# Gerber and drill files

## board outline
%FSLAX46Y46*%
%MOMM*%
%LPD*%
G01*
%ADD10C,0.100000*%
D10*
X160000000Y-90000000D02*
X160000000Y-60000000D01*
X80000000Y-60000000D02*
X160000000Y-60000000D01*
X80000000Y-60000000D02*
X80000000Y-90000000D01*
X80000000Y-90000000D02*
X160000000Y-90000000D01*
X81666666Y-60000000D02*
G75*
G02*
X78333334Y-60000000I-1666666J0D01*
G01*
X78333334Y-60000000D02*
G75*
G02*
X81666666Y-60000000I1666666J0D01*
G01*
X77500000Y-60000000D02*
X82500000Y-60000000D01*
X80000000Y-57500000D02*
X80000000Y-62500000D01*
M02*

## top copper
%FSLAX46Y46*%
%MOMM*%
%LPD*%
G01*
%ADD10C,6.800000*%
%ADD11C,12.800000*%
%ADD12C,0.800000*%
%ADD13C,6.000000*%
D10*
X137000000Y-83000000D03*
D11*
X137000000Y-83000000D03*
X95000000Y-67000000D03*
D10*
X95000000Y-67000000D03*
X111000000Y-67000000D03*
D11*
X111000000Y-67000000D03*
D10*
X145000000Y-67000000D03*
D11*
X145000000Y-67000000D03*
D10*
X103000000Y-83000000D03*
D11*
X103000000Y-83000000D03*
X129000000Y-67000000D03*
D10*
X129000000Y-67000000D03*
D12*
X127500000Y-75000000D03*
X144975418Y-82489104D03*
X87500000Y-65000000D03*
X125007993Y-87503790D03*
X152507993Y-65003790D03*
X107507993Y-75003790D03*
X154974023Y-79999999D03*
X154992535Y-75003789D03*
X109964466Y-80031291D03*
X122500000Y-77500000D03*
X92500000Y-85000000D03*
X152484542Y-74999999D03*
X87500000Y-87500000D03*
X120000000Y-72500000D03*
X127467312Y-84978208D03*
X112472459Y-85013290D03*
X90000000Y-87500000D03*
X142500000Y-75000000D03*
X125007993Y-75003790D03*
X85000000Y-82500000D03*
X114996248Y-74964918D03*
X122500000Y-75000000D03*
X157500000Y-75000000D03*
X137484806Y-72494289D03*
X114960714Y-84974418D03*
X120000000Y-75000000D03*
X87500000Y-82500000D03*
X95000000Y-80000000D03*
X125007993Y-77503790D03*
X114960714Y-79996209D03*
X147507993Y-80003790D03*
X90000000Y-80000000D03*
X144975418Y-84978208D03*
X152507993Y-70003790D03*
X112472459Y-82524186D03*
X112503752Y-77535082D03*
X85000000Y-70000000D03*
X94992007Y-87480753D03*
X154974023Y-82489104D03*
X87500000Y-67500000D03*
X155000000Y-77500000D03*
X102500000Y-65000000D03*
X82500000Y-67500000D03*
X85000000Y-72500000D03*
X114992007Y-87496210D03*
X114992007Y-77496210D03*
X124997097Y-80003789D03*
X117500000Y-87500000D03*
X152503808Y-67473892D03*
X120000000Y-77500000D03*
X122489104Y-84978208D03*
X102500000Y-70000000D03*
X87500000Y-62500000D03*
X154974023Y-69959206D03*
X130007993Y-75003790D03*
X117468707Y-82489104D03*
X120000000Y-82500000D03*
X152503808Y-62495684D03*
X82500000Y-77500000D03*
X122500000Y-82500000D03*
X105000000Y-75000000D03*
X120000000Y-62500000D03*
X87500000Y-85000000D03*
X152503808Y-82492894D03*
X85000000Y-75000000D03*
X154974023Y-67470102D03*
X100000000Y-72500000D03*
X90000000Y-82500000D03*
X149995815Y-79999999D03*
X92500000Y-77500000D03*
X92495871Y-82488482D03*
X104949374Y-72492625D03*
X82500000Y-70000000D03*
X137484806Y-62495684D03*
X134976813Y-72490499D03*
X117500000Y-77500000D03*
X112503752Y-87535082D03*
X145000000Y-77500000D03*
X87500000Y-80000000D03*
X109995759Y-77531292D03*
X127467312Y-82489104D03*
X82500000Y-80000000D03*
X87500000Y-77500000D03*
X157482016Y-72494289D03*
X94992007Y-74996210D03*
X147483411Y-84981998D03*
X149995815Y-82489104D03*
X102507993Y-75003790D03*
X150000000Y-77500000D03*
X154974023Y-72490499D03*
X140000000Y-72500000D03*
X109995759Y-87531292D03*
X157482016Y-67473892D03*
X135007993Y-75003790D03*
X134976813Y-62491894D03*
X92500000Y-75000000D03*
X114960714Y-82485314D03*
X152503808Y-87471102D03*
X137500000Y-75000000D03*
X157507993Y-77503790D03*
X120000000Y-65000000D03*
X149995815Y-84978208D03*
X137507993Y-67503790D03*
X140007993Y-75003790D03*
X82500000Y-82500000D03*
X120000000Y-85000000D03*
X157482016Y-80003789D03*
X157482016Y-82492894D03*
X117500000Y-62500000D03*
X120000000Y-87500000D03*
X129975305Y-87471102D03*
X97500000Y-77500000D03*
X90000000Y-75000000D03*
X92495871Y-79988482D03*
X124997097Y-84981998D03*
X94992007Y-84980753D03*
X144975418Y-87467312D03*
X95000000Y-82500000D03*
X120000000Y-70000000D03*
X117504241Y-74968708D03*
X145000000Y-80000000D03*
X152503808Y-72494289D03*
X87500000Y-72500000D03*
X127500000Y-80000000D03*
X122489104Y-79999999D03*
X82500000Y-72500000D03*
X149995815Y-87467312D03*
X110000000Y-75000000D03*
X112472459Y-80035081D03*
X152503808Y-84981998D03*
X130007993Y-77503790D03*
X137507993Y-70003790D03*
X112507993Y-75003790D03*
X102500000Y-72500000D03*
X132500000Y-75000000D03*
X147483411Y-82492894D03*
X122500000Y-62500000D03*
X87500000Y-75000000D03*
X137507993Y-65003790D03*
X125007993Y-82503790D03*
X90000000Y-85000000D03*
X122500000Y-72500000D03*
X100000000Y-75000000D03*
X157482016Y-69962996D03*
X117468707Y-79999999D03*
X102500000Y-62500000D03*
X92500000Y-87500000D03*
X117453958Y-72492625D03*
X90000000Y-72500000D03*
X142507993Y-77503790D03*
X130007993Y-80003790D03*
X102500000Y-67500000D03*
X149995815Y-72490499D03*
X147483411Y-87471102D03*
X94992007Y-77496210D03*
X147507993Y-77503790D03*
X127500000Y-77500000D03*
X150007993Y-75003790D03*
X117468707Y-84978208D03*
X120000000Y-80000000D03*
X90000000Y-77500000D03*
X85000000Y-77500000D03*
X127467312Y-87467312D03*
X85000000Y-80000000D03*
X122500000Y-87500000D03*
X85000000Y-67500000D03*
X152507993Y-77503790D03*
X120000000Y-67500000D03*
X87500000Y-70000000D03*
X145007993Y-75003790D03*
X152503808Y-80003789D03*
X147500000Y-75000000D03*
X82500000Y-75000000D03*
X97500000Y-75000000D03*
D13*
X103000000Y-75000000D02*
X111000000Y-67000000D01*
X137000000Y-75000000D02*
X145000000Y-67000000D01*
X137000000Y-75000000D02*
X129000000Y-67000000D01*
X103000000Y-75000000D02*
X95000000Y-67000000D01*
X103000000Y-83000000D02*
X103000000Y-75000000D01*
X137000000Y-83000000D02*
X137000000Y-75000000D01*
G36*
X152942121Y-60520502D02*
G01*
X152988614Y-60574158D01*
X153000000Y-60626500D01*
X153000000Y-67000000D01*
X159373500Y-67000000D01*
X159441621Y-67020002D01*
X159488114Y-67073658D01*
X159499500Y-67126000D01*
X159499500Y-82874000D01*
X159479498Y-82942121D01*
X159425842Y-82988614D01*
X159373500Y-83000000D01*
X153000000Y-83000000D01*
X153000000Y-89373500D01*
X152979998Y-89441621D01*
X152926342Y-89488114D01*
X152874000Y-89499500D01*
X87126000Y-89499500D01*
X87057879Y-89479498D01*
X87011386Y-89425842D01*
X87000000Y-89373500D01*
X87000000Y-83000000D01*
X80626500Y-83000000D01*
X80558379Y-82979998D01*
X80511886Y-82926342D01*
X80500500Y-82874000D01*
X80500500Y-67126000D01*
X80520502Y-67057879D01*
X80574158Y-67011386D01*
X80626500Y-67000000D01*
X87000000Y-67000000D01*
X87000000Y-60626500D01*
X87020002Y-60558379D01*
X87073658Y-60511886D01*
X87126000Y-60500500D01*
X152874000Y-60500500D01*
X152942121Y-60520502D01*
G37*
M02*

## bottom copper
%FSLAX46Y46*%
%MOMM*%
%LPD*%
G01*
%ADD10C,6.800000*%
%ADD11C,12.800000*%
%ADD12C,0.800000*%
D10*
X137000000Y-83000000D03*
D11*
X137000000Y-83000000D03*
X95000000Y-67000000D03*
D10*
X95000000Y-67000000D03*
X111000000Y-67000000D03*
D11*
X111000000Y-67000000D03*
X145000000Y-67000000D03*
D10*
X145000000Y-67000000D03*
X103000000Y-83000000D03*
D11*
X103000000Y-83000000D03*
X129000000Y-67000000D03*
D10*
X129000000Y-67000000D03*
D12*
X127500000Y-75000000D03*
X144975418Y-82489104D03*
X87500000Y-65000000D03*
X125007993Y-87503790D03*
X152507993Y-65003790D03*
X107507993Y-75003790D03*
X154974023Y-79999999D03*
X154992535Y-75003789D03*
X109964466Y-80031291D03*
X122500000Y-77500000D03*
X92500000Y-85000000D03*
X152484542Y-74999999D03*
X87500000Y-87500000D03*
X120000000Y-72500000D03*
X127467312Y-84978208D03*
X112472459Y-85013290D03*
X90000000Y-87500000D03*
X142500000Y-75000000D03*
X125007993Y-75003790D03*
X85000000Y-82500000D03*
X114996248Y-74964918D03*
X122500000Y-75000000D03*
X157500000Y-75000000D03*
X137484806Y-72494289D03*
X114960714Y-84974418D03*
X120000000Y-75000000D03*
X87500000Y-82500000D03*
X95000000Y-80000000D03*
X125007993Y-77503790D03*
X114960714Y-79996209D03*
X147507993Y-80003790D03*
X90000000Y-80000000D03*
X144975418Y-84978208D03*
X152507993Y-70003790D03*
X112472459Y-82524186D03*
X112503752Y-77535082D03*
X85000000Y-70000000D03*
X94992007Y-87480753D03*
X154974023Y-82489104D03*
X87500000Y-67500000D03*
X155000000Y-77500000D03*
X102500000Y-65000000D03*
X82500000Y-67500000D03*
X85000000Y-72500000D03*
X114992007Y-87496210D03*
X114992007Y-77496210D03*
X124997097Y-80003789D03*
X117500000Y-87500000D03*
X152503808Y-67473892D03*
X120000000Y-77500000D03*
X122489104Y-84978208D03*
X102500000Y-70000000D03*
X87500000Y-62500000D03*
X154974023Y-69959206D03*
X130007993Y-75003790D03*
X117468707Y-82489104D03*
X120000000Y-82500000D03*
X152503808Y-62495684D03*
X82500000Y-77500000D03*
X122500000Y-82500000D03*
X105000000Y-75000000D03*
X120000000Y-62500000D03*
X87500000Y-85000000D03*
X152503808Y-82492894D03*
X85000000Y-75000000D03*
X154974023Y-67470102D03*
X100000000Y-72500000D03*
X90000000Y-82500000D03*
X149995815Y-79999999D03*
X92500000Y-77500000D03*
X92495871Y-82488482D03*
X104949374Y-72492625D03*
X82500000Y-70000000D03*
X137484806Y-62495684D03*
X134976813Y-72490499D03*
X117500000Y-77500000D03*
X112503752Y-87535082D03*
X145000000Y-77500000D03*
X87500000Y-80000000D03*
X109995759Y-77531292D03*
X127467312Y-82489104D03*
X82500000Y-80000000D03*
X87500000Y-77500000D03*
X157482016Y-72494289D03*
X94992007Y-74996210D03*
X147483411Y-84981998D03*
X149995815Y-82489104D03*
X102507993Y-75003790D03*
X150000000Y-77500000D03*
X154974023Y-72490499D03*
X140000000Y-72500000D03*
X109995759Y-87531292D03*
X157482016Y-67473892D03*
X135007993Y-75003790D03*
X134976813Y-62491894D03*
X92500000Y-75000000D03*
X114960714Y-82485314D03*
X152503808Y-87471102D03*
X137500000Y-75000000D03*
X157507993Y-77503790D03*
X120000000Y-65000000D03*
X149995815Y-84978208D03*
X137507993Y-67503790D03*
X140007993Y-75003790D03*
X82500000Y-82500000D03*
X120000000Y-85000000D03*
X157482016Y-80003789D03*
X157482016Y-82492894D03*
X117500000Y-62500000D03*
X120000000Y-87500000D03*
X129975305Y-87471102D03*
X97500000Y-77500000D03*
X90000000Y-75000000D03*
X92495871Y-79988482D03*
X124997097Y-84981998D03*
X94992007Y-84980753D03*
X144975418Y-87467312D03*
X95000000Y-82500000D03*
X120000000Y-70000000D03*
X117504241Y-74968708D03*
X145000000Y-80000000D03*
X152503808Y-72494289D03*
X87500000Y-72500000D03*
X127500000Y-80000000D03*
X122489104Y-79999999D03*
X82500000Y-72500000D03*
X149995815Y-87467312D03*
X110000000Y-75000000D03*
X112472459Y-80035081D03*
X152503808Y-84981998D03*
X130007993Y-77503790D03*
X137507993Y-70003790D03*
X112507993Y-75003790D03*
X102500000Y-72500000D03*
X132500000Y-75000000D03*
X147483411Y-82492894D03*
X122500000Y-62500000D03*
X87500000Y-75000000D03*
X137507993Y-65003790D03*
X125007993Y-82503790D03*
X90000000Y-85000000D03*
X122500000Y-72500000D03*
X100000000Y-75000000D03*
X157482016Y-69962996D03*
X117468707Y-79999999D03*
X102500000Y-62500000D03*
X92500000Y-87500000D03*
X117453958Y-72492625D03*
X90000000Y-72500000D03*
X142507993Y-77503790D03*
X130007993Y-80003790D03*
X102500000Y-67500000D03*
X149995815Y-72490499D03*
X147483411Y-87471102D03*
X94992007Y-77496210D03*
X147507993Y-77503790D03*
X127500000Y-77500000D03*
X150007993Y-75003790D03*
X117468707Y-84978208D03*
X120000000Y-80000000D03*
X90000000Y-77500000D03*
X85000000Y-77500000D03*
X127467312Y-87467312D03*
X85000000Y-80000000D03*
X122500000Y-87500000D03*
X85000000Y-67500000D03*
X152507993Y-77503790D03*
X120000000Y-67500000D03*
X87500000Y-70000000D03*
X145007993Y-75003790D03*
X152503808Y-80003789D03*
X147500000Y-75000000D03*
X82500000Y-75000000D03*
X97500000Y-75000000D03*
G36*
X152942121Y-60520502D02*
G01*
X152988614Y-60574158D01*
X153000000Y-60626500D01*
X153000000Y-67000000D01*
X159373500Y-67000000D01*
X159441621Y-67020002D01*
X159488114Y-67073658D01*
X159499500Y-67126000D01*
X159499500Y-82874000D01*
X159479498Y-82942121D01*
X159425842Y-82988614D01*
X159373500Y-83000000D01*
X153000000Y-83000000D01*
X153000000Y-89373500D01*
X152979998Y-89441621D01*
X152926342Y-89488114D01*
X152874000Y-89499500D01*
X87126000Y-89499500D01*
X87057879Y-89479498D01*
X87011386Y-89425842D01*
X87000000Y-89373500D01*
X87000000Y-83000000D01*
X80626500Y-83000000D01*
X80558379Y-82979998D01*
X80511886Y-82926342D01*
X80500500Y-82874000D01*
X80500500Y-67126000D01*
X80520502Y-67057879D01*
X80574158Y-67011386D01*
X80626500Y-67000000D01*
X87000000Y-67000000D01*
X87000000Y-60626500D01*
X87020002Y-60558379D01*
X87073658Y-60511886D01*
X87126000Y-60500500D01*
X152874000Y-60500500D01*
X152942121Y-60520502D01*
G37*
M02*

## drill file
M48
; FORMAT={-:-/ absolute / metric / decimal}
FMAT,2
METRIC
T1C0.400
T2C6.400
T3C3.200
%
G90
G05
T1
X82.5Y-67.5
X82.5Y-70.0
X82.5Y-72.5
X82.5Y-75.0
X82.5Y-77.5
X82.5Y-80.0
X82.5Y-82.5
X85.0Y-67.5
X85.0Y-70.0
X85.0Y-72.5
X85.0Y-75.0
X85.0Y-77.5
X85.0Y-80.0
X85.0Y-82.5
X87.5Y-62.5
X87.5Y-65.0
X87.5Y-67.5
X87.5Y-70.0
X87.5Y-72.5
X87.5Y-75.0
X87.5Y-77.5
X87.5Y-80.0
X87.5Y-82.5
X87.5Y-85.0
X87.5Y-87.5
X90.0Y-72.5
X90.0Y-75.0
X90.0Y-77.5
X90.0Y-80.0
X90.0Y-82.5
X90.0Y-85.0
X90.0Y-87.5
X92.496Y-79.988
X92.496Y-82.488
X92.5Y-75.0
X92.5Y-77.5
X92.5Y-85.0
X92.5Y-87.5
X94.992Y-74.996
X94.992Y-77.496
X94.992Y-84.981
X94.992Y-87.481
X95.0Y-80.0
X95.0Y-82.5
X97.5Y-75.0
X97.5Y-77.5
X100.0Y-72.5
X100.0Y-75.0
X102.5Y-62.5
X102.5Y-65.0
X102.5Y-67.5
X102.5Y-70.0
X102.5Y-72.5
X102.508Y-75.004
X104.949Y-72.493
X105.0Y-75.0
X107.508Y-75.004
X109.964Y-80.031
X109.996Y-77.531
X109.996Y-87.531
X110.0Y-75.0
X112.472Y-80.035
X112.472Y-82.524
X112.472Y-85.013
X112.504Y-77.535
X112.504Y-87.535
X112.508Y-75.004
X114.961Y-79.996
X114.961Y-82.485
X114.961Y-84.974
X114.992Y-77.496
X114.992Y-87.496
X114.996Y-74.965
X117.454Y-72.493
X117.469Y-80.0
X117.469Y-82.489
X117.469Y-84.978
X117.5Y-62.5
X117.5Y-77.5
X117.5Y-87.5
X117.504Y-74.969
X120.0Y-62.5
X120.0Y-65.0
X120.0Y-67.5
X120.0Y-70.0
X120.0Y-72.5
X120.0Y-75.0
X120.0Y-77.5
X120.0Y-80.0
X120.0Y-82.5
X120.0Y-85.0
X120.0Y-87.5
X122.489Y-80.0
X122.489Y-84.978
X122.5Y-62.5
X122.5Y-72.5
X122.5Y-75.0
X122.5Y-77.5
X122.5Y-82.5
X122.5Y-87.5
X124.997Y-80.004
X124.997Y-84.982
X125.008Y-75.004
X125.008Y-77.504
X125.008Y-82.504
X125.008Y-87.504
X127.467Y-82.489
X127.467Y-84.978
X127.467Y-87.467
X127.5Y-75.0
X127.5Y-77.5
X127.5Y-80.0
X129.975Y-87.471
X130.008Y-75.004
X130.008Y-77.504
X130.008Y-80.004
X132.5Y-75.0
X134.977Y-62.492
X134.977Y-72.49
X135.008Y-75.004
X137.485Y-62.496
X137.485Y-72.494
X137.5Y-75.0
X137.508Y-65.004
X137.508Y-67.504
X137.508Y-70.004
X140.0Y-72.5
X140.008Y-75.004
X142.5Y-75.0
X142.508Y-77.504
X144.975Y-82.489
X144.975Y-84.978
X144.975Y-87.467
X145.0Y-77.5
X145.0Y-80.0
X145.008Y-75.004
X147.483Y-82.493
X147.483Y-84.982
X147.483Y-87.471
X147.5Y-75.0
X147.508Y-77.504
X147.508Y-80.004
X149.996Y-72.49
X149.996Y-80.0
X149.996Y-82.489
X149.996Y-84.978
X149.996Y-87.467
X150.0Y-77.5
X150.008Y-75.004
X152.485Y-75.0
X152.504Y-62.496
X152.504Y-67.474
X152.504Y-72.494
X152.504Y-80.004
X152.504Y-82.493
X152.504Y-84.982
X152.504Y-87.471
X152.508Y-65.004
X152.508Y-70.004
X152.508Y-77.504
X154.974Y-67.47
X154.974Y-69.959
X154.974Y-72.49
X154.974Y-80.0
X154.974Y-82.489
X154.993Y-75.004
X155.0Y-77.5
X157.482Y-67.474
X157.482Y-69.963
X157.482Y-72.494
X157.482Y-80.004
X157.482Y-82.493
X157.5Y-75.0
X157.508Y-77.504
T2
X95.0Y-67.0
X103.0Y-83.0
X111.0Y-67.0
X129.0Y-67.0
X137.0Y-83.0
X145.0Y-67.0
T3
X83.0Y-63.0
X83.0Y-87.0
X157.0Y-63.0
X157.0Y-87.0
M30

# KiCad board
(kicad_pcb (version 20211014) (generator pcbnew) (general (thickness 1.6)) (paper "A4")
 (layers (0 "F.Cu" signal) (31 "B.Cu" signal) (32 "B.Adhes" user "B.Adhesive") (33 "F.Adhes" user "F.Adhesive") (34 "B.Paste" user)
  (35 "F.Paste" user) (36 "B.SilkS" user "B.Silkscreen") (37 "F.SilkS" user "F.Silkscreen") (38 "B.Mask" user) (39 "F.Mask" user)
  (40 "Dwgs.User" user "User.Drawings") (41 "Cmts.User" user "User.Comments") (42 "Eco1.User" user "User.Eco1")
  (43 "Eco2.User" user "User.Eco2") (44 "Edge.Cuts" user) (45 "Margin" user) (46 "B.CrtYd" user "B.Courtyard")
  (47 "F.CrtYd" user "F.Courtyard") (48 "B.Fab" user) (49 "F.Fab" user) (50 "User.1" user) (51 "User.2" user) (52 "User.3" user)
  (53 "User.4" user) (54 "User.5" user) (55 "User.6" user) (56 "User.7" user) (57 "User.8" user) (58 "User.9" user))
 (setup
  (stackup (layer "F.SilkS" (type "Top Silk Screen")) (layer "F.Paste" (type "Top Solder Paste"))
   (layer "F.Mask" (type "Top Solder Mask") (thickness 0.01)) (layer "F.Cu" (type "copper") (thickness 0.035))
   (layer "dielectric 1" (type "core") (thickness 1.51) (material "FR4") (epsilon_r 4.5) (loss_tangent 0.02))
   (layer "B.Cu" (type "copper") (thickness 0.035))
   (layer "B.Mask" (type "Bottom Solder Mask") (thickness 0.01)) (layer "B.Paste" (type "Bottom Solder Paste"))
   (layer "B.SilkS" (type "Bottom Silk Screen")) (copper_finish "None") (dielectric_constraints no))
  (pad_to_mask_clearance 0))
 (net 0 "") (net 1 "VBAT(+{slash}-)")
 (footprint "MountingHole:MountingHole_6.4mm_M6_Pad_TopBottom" (layer "F.Cu") (at 137 83 90)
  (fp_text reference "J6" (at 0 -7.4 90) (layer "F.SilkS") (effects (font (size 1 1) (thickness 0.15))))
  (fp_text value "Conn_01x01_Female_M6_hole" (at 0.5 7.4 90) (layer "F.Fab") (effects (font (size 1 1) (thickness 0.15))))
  (pad "1" thru_hole circle locked (at 0 0 90) (size 6.8 6.8) (drill 6.4) (layers *.Cu *.Mask) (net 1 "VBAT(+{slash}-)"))
  (pad "1" connect circle locked (at 0 0 90) (size 12.8 12.8) (layers "F.Cu" "F.Mask") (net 1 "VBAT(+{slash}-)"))
  (pad "1" connect circle locked (at 0 0 90) (size 12.8 12.8) (layers "B.Cu" "B.Mask") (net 1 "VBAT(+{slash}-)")))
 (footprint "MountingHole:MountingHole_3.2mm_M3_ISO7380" (layer "F.Cu") (at 157 87)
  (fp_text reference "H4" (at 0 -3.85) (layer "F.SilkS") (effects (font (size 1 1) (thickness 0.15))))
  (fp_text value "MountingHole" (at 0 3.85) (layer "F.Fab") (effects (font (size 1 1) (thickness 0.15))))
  (pad "" np_thru_hole circle locked (at 0 0) (size 3.2 3.2) (drill 3.2) (layers *.Cu *.Mask)))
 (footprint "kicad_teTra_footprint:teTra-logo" (layer "F.Cu") (at 86 75)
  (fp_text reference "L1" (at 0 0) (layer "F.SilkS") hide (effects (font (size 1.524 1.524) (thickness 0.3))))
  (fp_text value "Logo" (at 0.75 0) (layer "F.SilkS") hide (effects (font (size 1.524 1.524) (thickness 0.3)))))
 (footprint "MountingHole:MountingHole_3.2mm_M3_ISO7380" (layer "F.Cu") (at 83 87)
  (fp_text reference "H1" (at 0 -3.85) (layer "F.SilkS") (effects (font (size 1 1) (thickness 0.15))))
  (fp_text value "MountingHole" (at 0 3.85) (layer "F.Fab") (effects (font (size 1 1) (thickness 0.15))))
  (pad "" np_thru_hole circle locked (at 0 0) (size 3.2 3.2) (drill 3.2) (layers *.Cu *.Mask)))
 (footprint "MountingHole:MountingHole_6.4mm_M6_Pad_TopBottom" (layer "F.Cu") (at 95 67 90)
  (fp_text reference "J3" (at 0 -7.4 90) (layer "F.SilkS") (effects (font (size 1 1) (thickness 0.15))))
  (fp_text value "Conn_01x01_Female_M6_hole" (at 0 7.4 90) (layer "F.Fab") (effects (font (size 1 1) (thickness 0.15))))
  (pad "1" connect circle locked (at 0 0 90) (size 12.8 12.8) (layers "B.Cu" "B.Mask") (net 1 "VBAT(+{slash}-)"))
  (pad "1" connect circle locked (at 0 0 90) (size 12.8 12.8) (layers "F.Cu" "F.Mask") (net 1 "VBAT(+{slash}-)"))
  (pad "1" thru_hole circle locked (at 0 0 90) (size 6.8 6.8) (drill 6.4) (layers *.Cu *.Mask) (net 1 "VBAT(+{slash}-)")))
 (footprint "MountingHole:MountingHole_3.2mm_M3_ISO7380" (layer "F.Cu") (at 83 63)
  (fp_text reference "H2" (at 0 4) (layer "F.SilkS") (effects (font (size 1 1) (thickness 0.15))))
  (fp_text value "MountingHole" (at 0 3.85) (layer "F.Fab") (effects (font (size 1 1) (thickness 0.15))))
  (pad "" np_thru_hole circle locked (at 0 0) (size 3.2 3.2) (drill 3.2) (layers *.Cu *.Mask)))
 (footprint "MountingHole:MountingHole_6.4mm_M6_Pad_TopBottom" (layer "F.Cu") (at 111 67 90)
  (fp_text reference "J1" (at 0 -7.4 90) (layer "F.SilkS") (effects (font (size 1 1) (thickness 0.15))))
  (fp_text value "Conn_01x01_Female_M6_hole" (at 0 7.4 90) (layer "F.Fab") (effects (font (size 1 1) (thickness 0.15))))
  (pad "1" thru_hole circle locked (at 0 0 90) (size 6.8 6.8) (drill 6.4) (layers *.Cu *.Mask) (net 1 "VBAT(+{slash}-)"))
  (pad "1" connect circle locked (at 0 0 90) (size 12.8 12.8) (layers "F.Cu" "F.Mask") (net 1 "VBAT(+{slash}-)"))
  (pad "1" connect circle locked (at 0 0 90) (size 12.8 12.8) (layers "B.Cu" "B.Mask") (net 1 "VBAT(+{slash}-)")))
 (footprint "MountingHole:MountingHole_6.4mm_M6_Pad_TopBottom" (layer "F.Cu") (at 145 67 90)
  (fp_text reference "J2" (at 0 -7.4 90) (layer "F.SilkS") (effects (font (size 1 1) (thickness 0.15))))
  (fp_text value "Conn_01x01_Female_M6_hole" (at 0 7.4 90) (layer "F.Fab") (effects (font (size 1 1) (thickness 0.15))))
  (pad "1" connect circle locked (at 0 0 90) (size 12.8 12.8) (layers "B.Cu" "B.Mask") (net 1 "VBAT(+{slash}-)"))
  (pad "1" thru_hole circle locked (at 0 0 90) (size 6.8 6.8) (drill 6.4) (layers *.Cu *.Mask) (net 1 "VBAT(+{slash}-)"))
  (pad "1" connect circle locked (at 0 0 90) (size 12.8 12.8) (layers "F.Cu" "F.Mask") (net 1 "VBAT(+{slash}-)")))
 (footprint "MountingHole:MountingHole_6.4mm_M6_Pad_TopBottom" (layer "F.Cu") (at 103 83 90)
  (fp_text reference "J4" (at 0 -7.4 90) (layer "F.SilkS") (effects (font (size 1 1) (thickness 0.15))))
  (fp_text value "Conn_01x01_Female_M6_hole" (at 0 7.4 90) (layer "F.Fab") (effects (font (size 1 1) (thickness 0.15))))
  (pad "1" thru_hole circle locked (at 0 0 90) (size 6.8 6.8) (drill 6.4) (layers *.Cu *.Mask) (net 1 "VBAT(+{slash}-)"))
  (pad "1" connect circle locked (at 0 0 90) (size 12.8 12.8) (layers "B.Cu" "B.Mask") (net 1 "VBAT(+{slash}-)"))
  (pad "1" connect circle locked (at 0 0 90) (size 12.8 12.8) (layers "F.Cu" "F.Mask") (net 1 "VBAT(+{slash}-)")))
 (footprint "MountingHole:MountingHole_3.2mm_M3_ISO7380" (layer "F.Cu") (at 157 63)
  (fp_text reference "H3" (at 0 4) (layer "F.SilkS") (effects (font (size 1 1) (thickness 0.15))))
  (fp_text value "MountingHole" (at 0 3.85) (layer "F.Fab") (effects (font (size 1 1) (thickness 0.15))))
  (pad "" np_thru_hole circle locked (at 0 0) (size 3.2 3.2) (drill 3.2) (layers *.Cu *.Mask)))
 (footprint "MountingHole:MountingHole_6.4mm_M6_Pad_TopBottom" (layer "F.Cu") (at 129 67 90)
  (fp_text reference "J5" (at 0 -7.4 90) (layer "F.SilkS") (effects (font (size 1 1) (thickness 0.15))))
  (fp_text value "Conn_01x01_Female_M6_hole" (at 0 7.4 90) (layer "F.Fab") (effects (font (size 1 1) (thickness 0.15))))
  (pad "1" connect circle locked (at 0 0 90) (size 12.8 12.8) (layers "F.Cu" "F.Mask") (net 1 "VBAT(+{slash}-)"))
  (pad "1" connect circle locked (at 0 0 90) (size 12.8 12.8) (layers "B.Cu" "B.Mask") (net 1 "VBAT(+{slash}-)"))
  (pad "1" thru_hole circle locked (at 0 0 90) (size 6.8 6.8) (drill 6.4) (layers *.Cu *.Mask) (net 1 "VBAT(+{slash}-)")))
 (gr_line (start 160 90) (end 160 60) (layer "Edge.Cuts") (width 0.1))
 (gr_line (start 80 60) (end 160 60) (layer "Edge.Cuts") (width 0.1))
 (gr_line (start 80 60) (end 80 90) (layer "Edge.Cuts") (width 0.1))
 (gr_line (start 80 90) (end 160 90) (layer "Edge.Cuts") (width 0.1))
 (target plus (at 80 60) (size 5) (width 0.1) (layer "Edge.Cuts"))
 (segment (start 103 75) (end 111 67) (width 6) (layer "F.Cu") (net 1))
 (segment (start 137 75) (end 145 67) (width 6) (layer "F.Cu") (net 1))
 (segment (start 137 75) (end 129 67) (width 6) (layer "F.Cu") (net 1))
 (segment (start 103 75) (end 95 67) (width 6) (layer "F.Cu") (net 1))
 (segment (start 103 83) (end 103 75) (width 6) (layer "F.Cu") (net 1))
 (segment (start 137 83) (end 137 75) (width 6) (layer "F.Cu") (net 1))
 (via (at 127.5 75) (size 0.8) (drill 0.4) (layers "F.Cu" "B.Cu") (free) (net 1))
 (via (at 144.975418 82.489104) (size 0.8) (drill 0.4) (layers "F.Cu" "B.Cu") (free) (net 1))
 (via (at 87.5 65) (size 0.8) (drill 0.4) (layers "F.Cu" "B.Cu") (free) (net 1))
 (via (at 125.007993 87.50379) (size 0.8) (drill 0.4) (layers "F.Cu" "B.Cu") (free) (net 1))
 (via (at 152.507993 65.00379) (size 0.8) (drill 0.4) (layers "F.Cu" "B.Cu") (free) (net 1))
 (via (at 107.507993 75.00379) (size 0.8) (drill 0.4) (layers "F.Cu" "B.Cu") (free) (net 1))
 (via (at 154.974023 79.999999) (size 0.8) (drill 0.4) (layers "F.Cu" "B.Cu") (free) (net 1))
 (via (at 154.992535 75.003789) (size 0.8) (drill 0.4) (layers "F.Cu" "B.Cu") (free) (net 1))
 (via (at 109.964466 80.031291) (size 0.8) (drill 0.4) (layers "F.Cu" "B.Cu") (free) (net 1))
 (via (at 122.5 77.5) (size 0.8) (drill 0.4) (layers "F.Cu" "B.Cu") (free) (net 1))
 (via (at 92.5 85) (size 0.8) (drill 0.4) (layers "F.Cu" "B.Cu") (free) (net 1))
 (via (at 152.484542 74.999999) (size 0.8) (drill 0.4) (layers "F.Cu" "B.Cu") (free) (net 1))
 (via (at 87.5 87.5) (size 0.8) (drill 0.4) (layers "F.Cu" "B.Cu") (free) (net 1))
 (via (at 120 72.5) (size 0.8) (drill 0.4) (layers "F.Cu" "B.Cu") (free) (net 1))
 (via (at 127.467312 84.978208) (size 0.8) (drill 0.4) (layers "F.Cu" "B.Cu") (free) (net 1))
 (via (at 112.472459 85.01329) (size 0.8) (drill 0.4) (layers "F.Cu" "B.Cu") (free) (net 1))
 (via (at 90 87.5) (size 0.8) (drill 0.4) (layers "F.Cu" "B.Cu") (free) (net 1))
 (via (at 142.5 75) (size 0.8) (drill 0.4) (layers "F.Cu" "B.Cu") (free) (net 1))
 (via (at 125.007993 75.00379) (size 0.8) (drill 0.4) (layers "F.Cu" "B.Cu") (free) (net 1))
 (via (at 85 82.5) (size 0.8) (drill 0.4) (layers "F.Cu" "B.Cu") (free) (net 1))
 (via (at 114.996248 74.964918) (size 0.8) (drill 0.4) (layers "F.Cu" "B.Cu") (free) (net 1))
 (via (at 122.5 75) (size 0.8) (drill 0.4) (layers "F.Cu" "B.Cu") (free) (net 1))
 (via (at 157.5 75) (size 0.8) (drill 0.4) (layers "F.Cu" "B.Cu") (free) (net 1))
 (via (at 137.484806 72.494289) (size 0.8) (drill 0.4) (layers "F.Cu" "B.Cu") (free) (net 1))
 (via (at 114.960714 84.974418) (size 0.8) (drill 0.4) (layers "F.Cu" "B.Cu") (free) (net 1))
 (via (at 120 75) (size 0.8) (drill 0.4) (layers "F.Cu" "B.Cu") (free) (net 1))
 (via (at 87.5 82.5) (size 0.8) (drill 0.4) (layers "F.Cu" "B.Cu") (free) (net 1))
 (via (at 95 80) (size 0.8) (drill 0.4) (layers "F.Cu" "B.Cu") (free) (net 1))
 (via (at 125.007993 77.50379) (size 0.8) (drill 0.4) (layers "F.Cu" "B.Cu") (free) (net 1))
 (via (at 114.960714 79.996209) (size 0.8) (drill 0.4) (layers "F.Cu" "B.Cu") (free) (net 1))
 (via (at 147.507993 80.00379) (size 0.8) (drill 0.4) (layers "F.Cu" "B.Cu") (free) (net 1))
 (via (at 90 80) (size 0.8) (drill 0.4) (layers "F.Cu" "B.Cu") (free) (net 1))
 (via (at 144.975418 84.978208) (size 0.8) (drill 0.4) (layers "F.Cu" "B.Cu") (free) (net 1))
 (via (at 152.507993 70.00379) (size 0.8) (drill 0.4) (layers "F.Cu" "B.Cu") (free) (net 1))
 (via (at 112.472459 82.524186) (size 0.8) (drill 0.4) (layers "F.Cu" "B.Cu") (free) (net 1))
 (via (at 112.503752 77.535082) (size 0.8) (drill 0.4) (layers "F.Cu" "B.Cu") (free) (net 1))
 (via (at 85 70) (size 0.8) (drill 0.4) (layers "F.Cu" "B.Cu") (free) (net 1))
 (via (at 94.992007 87.480753) (size 0.8) (drill 0.4) (layers "F.Cu" "B.Cu") (free) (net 1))
 (via (at 154.974023 82.489104) (size 0.8) (drill 0.4) (layers "F.Cu" "B.Cu") (free) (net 1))
 (via (at 87.5 67.5) (size 0.8) (drill 0.4) (layers "F.Cu" "B.Cu") (free) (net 1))
 (via (at 155 77.5) (size 0.8) (drill 0.4) (layers "F.Cu" "B.Cu") (free) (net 1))
 (via (at 102.5 65) (size 0.8) (drill 0.4) (layers "F.Cu" "B.Cu") (free) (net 1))
 (via (at 82.5 67.5) (size 0.8) (drill 0.4) (layers "F.Cu" "B.Cu") (free) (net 1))
 (via (at 85 72.5) (size 0.8) (drill 0.4) (layers "F.Cu" "B.Cu") (free) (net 1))
 (via (at 114.992007 87.49621) (size 0.8) (drill 0.4) (layers "F.Cu" "B.Cu") (free) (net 1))
 (via (at 114.992007 77.49621) (size 0.8) (drill 0.4) (layers "F.Cu" "B.Cu") (free) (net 1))
 (via (at 124.997097 80.003789) (size 0.8) (drill 0.4) (layers "F.Cu" "B.Cu") (free) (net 1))
 (via (at 117.5 87.5) (size 0.8) (drill 0.4) (layers "F.Cu" "B.Cu") (free) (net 1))
 (via (at 152.503808 67.473892) (size 0.8) (drill 0.4) (layers "F.Cu" "B.Cu") (free) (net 1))
 (via (at 120 77.5) (size 0.8) (drill 0.4) (layers "F.Cu" "B.Cu") (free) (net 1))
 (via (at 122.489104 84.978208) (size 0.8) (drill 0.4) (layers "F.Cu" "B.Cu") (free) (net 1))
 (via (at 102.5 70) (size 0.8) (drill 0.4) (layers "F.Cu" "B.Cu") (free) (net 1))
 (via (at 87.5 62.5) (size 0.8) (drill 0.4) (layers "F.Cu" "B.Cu") (free) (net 1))
 (via (at 154.974023 69.959206) (size 0.8) (drill 0.4) (layers "F.Cu" "B.Cu") (free) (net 1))
 (via (at 130.007993 75.00379) (size 0.8) (drill 0.4) (layers "F.Cu" "B.Cu") (free) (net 1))
 (via (at 117.468707 82.489104) (size 0.8) (drill 0.4) (layers "F.Cu" "B.Cu") (free) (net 1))
 (via (at 120 82.5) (size 0.8) (drill 0.4) (layers "F.Cu" "B.Cu") (free) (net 1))
 (via (at 152.503808 62.495684) (size 0.8) (drill 0.4) (layers "F.Cu" "B.Cu") (free) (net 1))
 (via (at 82.5 77.5) (size 0.8) (drill 0.4) (layers "F.Cu" "B.Cu") (free) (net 1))
 (via (at 122.5 82.5) (size 0.8) (drill 0.4) (layers "F.Cu" "B.Cu") (free) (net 1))
 (via (at 105 75) (size 0.8) (drill 0.4) (layers "F.Cu" "B.Cu") (free) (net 1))
 (via (at 120 62.5) (size 0.8) (drill 0.4) (layers "F.Cu" "B.Cu") (free) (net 1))
 (via (at 87.5 85) (size 0.8) (drill 0.4) (layers "F.Cu" "B.Cu") (free) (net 1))
 (via (at 152.503808 82.492894) (size 0.8) (drill 0.4) (layers "F.Cu" "B.Cu") (free) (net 1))
 (via (at 85 75) (size 0.8) (drill 0.4) (layers "F.Cu" "B.Cu") (free) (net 1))
 (via (at 154.974023 67.470102) (size 0.8) (drill 0.4) (layers "F.Cu" "B.Cu") (free) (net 1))
 (via (at 100 72.5) (size 0.8) (drill 0.4) (layers "F.Cu" "B.Cu") (free) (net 1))
 (via (at 90 82.5) (size 0.8) (drill 0.4) (layers "F.Cu" "B.Cu") (free) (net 1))
 (via (at 149.995815 79.999999) (size 0.8) (drill 0.4) (layers "F.Cu" "B.Cu") (free) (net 1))
 (via (at 92.5 77.5) (size 0.8) (drill 0.4) (layers "F.Cu" "B.Cu") (free) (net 1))
 (via (at 92.495871 82.488482) (size 0.8) (drill 0.4) (layers "F.Cu" "B.Cu") (free) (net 1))
 (via (at 104.949374 72.492625) (size 0.8) (drill 0.4) (layers "F.Cu" "B.Cu") (free) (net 1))
 (via (at 82.5 70) (size 0.8) (drill 0.4) (layers "F.Cu" "B.Cu") (free) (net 1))
 (via (at 137.484806 62.495684) (size 0.8) (drill 0.4) (layers "F.Cu" "B.Cu") (free) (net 1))
 (via (at 134.976813 72.490499) (size 0.8) (drill 0.4) (layers "F.Cu" "B.Cu") (free) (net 1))
 (via (at 117.5 77.5) (size 0.8) (drill 0.4) (layers "F.Cu" "B.Cu") (free) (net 1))
 (via (at 112.503752 87.535082) (size 0.8) (drill 0.4) (layers "F.Cu" "B.Cu") (free) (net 1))
 (via (at 145 77.5) (size 0.8) (drill 0.4) (layers "F.Cu" "B.Cu") (free) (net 1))
 (via (at 87.5 80) (size 0.8) (drill 0.4) (layers "F.Cu" "B.Cu") (free) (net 1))
 (via (at 109.995759 77.531292) (size 0.8) (drill 0.4) (layers "F.Cu" "B.Cu") (free) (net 1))
 (via (at 127.467312 82.489104) (size 0.8) (drill 0.4) (layers "F.Cu" "B.Cu") (free) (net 1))
 (via (at 82.5 80) (size 0.8) (drill 0.4) (layers "F.Cu" "B.Cu") (free) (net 1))
 (via (at 87.5 77.5) (size 0.8) (drill 0.4) (layers "F.Cu" "B.Cu") (free) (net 1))
 (via (at 157.482016 72.494289) (size 0.8) (drill 0.4) (layers "F.Cu" "B.Cu") (free) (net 1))
 (via (at 94.992007 74.99621) (size 0.8) (drill 0.4) (layers "F.Cu" "B.Cu") (free) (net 1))
 (via (at 147.483411 84.981998) (size 0.8) (drill 0.4) (layers "F.Cu" "B.Cu") (free) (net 1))
 (via (at 149.995815 82.489104) (size 0.8) (drill 0.4) (layers "F.Cu" "B.Cu") (free) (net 1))
 (via (at 102.507993 75.00379) (size 0.8) (drill 0.4) (layers "F.Cu" "B.Cu") (free) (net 1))
 (via (at 150 77.5) (size 0.8) (drill 0.4) (layers "F.Cu" "B.Cu") (free) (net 1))
 (via (at 154.974023 72.490499) (size 0.8) (drill 0.4) (layers "F.Cu" "B.Cu") (free) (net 1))
 (via (at 140 72.5) (size 0.8) (drill 0.4) (layers "F.Cu" "B.Cu") (free) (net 1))
 (via (at 109.995759 87.531292) (size 0.8) (drill 0.4) (layers "F.Cu" "B.Cu") (free) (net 1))
 (via (at 157.482016 67.473892) (size 0.8) (drill 0.4) (layers "F.Cu" "B.Cu") (free) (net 1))
 (via (at 135.007993 75.00379) (size 0.8) (drill 0.4) (layers "F.Cu" "B.Cu") (free) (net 1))
 (via (at 134.976813 62.491894) (size 0.8) (drill 0.4) (layers "F.Cu" "B.Cu") (free) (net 1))
 (via (at 92.5 75) (size 0.8) (drill 0.4) (layers "F.Cu" "B.Cu") (free) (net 1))
 (via (at 114.960714 82.485314) (size 0.8) (drill 0.4) (layers "F.Cu" "B.Cu") (free) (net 1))
 (via (at 152.503808 87.471102) (size 0.8) (drill 0.4) (layers "F.Cu" "B.Cu") (free) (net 1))
 (via (at 137.5 75) (size 0.8) (drill 0.4) (layers "F.Cu" "B.Cu") (free) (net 1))
 (via (at 157.507993 77.50379) (size 0.8) (drill 0.4) (layers "F.Cu" "B.Cu") (free) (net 1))
 (via (at 120 65) (size 0.8) (drill 0.4) (layers "F.Cu" "B.Cu") (free) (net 1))
 (via (at 149.995815 84.978208) (size 0.8) (drill 0.4) (layers "F.Cu" "B.Cu") (free) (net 1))
 (via (at 137.507993 67.50379) (size 0.8) (drill 0.4) (layers "F.Cu" "B.Cu") (free) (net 1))
 (via (at 140.007993 75.00379) (size 0.8) (drill 0.4) (layers "F.Cu" "B.Cu") (free) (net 1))
 (via (at 82.5 82.5) (size 0.8) (drill 0.4) (layers "F.Cu" "B.Cu") (free) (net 1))
 (via (at 120 85) (size 0.8) (drill 0.4) (layers "F.Cu" "B.Cu") (free) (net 1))
 (via (at 157.482016 80.003789) (size 0.8) (drill 0.4) (layers "F.Cu" "B.Cu") (free) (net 1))
 (via (at 157.482016 82.492894) (size 0.8) (drill 0.4) (layers "F.Cu" "B.Cu") (free) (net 1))
 (via (at 117.5 62.5) (size 0.8) (drill 0.4) (layers "F.Cu" "B.Cu") (free) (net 1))
 (via (at 120 87.5) (size 0.8) (drill 0.4) (layers "F.Cu" "B.Cu") (free) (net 1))
 (via (at 129.975305 87.471102) (size 0.8) (drill 0.4) (layers "F.Cu" "B.Cu") (free) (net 1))
 (via (at 97.5 77.5) (size 0.8) (drill 0.4) (layers "F.Cu" "B.Cu") (free) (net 1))
 (via (at 90 75) (size 0.8) (drill 0.4) (layers "F.Cu" "B.Cu") (free) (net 1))
 (via (at 92.495871 79.988482) (size 0.8) (drill 0.4) (layers "F.Cu" "B.Cu") (free) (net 1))
 (via (at 124.997097 84.981998) (size 0.8) (drill 0.4) (layers "F.Cu" "B.Cu") (free) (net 1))
 (via (at 94.992007 84.980753) (size 0.8) (drill 0.4) (layers "F.Cu" "B.Cu") (free) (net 1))
 (via (at 144.975418 87.467312) (size 0.8) (drill 0.4) (layers "F.Cu" "B.Cu") (free) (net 1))
 (via (at 95 82.5) (size 0.8) (drill 0.4) (layers "F.Cu" "B.Cu") (free) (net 1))
 (via (at 120 70) (size 0.8) (drill 0.4) (layers "F.Cu" "B.Cu") (free) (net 1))
 (via (at 117.504241 74.968708) (size 0.8) (drill 0.4) (layers "F.Cu" "B.Cu") (free) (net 1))
 (via (at 145 80) (size 0.8) (drill 0.4) (layers "F.Cu" "B.Cu") (free) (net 1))
 (via (at 152.503808 72.494289) (size 0.8) (drill 0.4) (layers "F.Cu" "B.Cu") (free) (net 1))
 (via (at 87.5 72.5) (size 0.8) (drill 0.4) (layers "F.Cu" "B.Cu") (free) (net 1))
 (via (at 127.5 80) (size 0.8) (drill 0.4) (layers "F.Cu" "B.Cu") (free) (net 1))
 (via (at 122.489104 79.999999) (size 0.8) (drill 0.4) (layers "F.Cu" "B.Cu") (free) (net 1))
 (via (at 82.5 72.5) (size 0.8) (drill 0.4) (layers "F.Cu" "B.Cu") (free) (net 1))
 (via (at 149.995815 87.467312) (size 0.8) (drill 0.4) (layers "F.Cu" "B.Cu") (free) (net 1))
 (via (at 110 75) (size 0.8) (drill 0.4) (layers "F.Cu" "B.Cu") (free) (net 1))
 (via (at 112.472459 80.035081) (size 0.8) (drill 0.4) (layers "F.Cu" "B.Cu") (free) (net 1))
 (via (at 152.503808 84.981998) (size 0.8) (drill 0.4) (layers "F.Cu" "B.Cu") (free) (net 1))
 (via (at 130.007993 77.50379) (size 0.8) (drill 0.4) (layers "F.Cu" "B.Cu") (free) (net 1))
 (via (at 137.507993 70.00379) (size 0.8) (drill 0.4) (layers "F.Cu" "B.Cu") (free) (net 1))
 (via (at 112.507993 75.00379) (size 0.8) (drill 0.4) (layers "F.Cu" "B.Cu") (free) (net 1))
 (via (at 102.5 72.5) (size 0.8) (drill 0.4) (layers "F.Cu" "B.Cu") (free) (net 1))
 (via (at 132.5 75) (size 0.8) (drill 0.4) (layers "F.Cu" "B.Cu") (free) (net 1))
 (via (at 147.483411 82.492894) (size 0.8) (drill 0.4) (layers "F.Cu" "B.Cu") (free) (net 1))
 (via (at 122.5 62.5) (size 0.8) (drill 0.4) (layers "F.Cu" "B.Cu") (free) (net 1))
 (via (at 87.5 75) (size 0.8) (drill 0.4) (layers "F.Cu" "B.Cu") (free) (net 1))
 (via (at 137.507993 65.00379) (size 0.8) (drill 0.4) (layers "F.Cu" "B.Cu") (free) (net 1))
 (via (at 125.007993 82.50379) (size 0.8) (drill 0.4) (layers "F.Cu" "B.Cu") (free) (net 1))
 (via (at 90 85) (size 0.8) (drill 0.4) (layers "F.Cu" "B.Cu") (free) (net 1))
 (via (at 122.5 72.5) (size 0.8) (drill 0.4) (layers "F.Cu" "B.Cu") (free) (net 1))
 (via (at 100 75) (size 0.8) (drill 0.4) (layers "F.Cu" "B.Cu") (free) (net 1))
 (via (at 157.482016 69.962996) (size 0.8) (drill 0.4) (layers "F.Cu" "B.Cu") (free) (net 1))
 (via (at 117.468707 79.999999) (size 0.8) (drill 0.4) (layers "F.Cu" "B.Cu") (free) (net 1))
 (via (at 102.5 62.5) (size 0.8) (drill 0.4) (layers "F.Cu" "B.Cu") (free) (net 1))
 (via (at 92.5 87.5) (size 0.8) (drill 0.4) (layers "F.Cu" "B.Cu") (free) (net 1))
 (via (at 117.453958 72.492625) (size 0.8) (drill 0.4) (layers "F.Cu" "B.Cu") (free) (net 1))
 (via (at 90 72.5) (size 0.8) (drill 0.4) (layers "F.Cu" "B.Cu") (free) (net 1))
 (via (at 142.507993 77.50379) (size 0.8) (drill 0.4) (layers "F.Cu" "B.Cu") (free) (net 1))
 (via (at 130.007993 80.00379) (size 0.8) (drill 0.4) (layers "F.Cu" "B.Cu") (free) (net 1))
 (via (at 102.5 67.5) (size 0.8) (drill 0.4) (layers "F.Cu" "B.Cu") (free) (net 1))
 (via (at 149.995815 72.490499) (size 0.8) (drill 0.4) (layers "F.Cu" "B.Cu") (free) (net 1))
 (via (at 147.483411 87.471102) (size 0.8) (drill 0.4) (layers "F.Cu" "B.Cu") (free) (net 1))
 (via (at 94.992007 77.49621) (size 0.8) (drill 0.4) (layers "F.Cu" "B.Cu") (free) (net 1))
 (via (at 147.507993 77.50379) (size 0.8) (drill 0.4) (layers "F.Cu" "B.Cu") (free) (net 1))
 (via (at 127.5 77.5) (size 0.8) (drill 0.4) (layers "F.Cu" "B.Cu") (free) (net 1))
 (via (at 150.007993 75.00379) (size 0.8) (drill 0.4) (layers "F.Cu" "B.Cu") (free) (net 1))
 (via (at 117.468707 84.978208) (size 0.8) (drill 0.4) (layers "F.Cu" "B.Cu") (free) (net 1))
 (via (at 120 80) (size 0.8) (drill 0.4) (layers "F.Cu" "B.Cu") (free) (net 1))
 (via (at 90 77.5) (size 0.8) (drill 0.4) (layers "F.Cu" "B.Cu") (free) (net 1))
 (via (at 85 77.5) (size 0.8) (drill 0.4) (layers "F.Cu" "B.Cu") (free) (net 1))
 (via (at 127.467312 87.467312) (size 0.8) (drill 0.4) (layers "F.Cu" "B.Cu") (free) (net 1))
 (via (at 85 80) (size 0.8) (drill 0.4) (layers "F.Cu" "B.Cu") (free) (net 1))
 (via (at 122.5 87.5) (size 0.8) (drill 0.4) (layers "F.Cu" "B.Cu") (free) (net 1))
 (via (at 85 67.5) (size 0.8) (drill 0.4) (layers "F.Cu" "B.Cu") (free) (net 1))
 (via (at 152.507993 77.50379) (size 0.8) (drill 0.4) (layers "F.Cu" "B.Cu") (free) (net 1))
 (via (at 120 67.5) (size 0.8) (drill 0.4) (layers "F.Cu" "B.Cu") (free) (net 1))
 (via (at 87.5 70) (size 0.8) (drill 0.4) (layers "F.Cu" "B.Cu") (free) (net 1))
 (via (at 145.007993 75.00379) (size 0.8) (drill 0.4) (layers "F.Cu" "B.Cu") (free) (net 1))
 (via (at 152.503808 80.003789) (size 0.8) (drill 0.4) (layers "F.Cu" "B.Cu") (free) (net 1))
 (via (at 147.5 75) (size 0.8) (drill 0.4) (layers "F.Cu" "B.Cu") (free) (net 1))
 (via (at 82.5 75) (size 0.8) (drill 0.4) (layers "F.Cu" "B.Cu") (free) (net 1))
 (via (at 97.5 75) (size 0.8) (drill 0.4) (layers "F.Cu" "B.Cu") (free) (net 1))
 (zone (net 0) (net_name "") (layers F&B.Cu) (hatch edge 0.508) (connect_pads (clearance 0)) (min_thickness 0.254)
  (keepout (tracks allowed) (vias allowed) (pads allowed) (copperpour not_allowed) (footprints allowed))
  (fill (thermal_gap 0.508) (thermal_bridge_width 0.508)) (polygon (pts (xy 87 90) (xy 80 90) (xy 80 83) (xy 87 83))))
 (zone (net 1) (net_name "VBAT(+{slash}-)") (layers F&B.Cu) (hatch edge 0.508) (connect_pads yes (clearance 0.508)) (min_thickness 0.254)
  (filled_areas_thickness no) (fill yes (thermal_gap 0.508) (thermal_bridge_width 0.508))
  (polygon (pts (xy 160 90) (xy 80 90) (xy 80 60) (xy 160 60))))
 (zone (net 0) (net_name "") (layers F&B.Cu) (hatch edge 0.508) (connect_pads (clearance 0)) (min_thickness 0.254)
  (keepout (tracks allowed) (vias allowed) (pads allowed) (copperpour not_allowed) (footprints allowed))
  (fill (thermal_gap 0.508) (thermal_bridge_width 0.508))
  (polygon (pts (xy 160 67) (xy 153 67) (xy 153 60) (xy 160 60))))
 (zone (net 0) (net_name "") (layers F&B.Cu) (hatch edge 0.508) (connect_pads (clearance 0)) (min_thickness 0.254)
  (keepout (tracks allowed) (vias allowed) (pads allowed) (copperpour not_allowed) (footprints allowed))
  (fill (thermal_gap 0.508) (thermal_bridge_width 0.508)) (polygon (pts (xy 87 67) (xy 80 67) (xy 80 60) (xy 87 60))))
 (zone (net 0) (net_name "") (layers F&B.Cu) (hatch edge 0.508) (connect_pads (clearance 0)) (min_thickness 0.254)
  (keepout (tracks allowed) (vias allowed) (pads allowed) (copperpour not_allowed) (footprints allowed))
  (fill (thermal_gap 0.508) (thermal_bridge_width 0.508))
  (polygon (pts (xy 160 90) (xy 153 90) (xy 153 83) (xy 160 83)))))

